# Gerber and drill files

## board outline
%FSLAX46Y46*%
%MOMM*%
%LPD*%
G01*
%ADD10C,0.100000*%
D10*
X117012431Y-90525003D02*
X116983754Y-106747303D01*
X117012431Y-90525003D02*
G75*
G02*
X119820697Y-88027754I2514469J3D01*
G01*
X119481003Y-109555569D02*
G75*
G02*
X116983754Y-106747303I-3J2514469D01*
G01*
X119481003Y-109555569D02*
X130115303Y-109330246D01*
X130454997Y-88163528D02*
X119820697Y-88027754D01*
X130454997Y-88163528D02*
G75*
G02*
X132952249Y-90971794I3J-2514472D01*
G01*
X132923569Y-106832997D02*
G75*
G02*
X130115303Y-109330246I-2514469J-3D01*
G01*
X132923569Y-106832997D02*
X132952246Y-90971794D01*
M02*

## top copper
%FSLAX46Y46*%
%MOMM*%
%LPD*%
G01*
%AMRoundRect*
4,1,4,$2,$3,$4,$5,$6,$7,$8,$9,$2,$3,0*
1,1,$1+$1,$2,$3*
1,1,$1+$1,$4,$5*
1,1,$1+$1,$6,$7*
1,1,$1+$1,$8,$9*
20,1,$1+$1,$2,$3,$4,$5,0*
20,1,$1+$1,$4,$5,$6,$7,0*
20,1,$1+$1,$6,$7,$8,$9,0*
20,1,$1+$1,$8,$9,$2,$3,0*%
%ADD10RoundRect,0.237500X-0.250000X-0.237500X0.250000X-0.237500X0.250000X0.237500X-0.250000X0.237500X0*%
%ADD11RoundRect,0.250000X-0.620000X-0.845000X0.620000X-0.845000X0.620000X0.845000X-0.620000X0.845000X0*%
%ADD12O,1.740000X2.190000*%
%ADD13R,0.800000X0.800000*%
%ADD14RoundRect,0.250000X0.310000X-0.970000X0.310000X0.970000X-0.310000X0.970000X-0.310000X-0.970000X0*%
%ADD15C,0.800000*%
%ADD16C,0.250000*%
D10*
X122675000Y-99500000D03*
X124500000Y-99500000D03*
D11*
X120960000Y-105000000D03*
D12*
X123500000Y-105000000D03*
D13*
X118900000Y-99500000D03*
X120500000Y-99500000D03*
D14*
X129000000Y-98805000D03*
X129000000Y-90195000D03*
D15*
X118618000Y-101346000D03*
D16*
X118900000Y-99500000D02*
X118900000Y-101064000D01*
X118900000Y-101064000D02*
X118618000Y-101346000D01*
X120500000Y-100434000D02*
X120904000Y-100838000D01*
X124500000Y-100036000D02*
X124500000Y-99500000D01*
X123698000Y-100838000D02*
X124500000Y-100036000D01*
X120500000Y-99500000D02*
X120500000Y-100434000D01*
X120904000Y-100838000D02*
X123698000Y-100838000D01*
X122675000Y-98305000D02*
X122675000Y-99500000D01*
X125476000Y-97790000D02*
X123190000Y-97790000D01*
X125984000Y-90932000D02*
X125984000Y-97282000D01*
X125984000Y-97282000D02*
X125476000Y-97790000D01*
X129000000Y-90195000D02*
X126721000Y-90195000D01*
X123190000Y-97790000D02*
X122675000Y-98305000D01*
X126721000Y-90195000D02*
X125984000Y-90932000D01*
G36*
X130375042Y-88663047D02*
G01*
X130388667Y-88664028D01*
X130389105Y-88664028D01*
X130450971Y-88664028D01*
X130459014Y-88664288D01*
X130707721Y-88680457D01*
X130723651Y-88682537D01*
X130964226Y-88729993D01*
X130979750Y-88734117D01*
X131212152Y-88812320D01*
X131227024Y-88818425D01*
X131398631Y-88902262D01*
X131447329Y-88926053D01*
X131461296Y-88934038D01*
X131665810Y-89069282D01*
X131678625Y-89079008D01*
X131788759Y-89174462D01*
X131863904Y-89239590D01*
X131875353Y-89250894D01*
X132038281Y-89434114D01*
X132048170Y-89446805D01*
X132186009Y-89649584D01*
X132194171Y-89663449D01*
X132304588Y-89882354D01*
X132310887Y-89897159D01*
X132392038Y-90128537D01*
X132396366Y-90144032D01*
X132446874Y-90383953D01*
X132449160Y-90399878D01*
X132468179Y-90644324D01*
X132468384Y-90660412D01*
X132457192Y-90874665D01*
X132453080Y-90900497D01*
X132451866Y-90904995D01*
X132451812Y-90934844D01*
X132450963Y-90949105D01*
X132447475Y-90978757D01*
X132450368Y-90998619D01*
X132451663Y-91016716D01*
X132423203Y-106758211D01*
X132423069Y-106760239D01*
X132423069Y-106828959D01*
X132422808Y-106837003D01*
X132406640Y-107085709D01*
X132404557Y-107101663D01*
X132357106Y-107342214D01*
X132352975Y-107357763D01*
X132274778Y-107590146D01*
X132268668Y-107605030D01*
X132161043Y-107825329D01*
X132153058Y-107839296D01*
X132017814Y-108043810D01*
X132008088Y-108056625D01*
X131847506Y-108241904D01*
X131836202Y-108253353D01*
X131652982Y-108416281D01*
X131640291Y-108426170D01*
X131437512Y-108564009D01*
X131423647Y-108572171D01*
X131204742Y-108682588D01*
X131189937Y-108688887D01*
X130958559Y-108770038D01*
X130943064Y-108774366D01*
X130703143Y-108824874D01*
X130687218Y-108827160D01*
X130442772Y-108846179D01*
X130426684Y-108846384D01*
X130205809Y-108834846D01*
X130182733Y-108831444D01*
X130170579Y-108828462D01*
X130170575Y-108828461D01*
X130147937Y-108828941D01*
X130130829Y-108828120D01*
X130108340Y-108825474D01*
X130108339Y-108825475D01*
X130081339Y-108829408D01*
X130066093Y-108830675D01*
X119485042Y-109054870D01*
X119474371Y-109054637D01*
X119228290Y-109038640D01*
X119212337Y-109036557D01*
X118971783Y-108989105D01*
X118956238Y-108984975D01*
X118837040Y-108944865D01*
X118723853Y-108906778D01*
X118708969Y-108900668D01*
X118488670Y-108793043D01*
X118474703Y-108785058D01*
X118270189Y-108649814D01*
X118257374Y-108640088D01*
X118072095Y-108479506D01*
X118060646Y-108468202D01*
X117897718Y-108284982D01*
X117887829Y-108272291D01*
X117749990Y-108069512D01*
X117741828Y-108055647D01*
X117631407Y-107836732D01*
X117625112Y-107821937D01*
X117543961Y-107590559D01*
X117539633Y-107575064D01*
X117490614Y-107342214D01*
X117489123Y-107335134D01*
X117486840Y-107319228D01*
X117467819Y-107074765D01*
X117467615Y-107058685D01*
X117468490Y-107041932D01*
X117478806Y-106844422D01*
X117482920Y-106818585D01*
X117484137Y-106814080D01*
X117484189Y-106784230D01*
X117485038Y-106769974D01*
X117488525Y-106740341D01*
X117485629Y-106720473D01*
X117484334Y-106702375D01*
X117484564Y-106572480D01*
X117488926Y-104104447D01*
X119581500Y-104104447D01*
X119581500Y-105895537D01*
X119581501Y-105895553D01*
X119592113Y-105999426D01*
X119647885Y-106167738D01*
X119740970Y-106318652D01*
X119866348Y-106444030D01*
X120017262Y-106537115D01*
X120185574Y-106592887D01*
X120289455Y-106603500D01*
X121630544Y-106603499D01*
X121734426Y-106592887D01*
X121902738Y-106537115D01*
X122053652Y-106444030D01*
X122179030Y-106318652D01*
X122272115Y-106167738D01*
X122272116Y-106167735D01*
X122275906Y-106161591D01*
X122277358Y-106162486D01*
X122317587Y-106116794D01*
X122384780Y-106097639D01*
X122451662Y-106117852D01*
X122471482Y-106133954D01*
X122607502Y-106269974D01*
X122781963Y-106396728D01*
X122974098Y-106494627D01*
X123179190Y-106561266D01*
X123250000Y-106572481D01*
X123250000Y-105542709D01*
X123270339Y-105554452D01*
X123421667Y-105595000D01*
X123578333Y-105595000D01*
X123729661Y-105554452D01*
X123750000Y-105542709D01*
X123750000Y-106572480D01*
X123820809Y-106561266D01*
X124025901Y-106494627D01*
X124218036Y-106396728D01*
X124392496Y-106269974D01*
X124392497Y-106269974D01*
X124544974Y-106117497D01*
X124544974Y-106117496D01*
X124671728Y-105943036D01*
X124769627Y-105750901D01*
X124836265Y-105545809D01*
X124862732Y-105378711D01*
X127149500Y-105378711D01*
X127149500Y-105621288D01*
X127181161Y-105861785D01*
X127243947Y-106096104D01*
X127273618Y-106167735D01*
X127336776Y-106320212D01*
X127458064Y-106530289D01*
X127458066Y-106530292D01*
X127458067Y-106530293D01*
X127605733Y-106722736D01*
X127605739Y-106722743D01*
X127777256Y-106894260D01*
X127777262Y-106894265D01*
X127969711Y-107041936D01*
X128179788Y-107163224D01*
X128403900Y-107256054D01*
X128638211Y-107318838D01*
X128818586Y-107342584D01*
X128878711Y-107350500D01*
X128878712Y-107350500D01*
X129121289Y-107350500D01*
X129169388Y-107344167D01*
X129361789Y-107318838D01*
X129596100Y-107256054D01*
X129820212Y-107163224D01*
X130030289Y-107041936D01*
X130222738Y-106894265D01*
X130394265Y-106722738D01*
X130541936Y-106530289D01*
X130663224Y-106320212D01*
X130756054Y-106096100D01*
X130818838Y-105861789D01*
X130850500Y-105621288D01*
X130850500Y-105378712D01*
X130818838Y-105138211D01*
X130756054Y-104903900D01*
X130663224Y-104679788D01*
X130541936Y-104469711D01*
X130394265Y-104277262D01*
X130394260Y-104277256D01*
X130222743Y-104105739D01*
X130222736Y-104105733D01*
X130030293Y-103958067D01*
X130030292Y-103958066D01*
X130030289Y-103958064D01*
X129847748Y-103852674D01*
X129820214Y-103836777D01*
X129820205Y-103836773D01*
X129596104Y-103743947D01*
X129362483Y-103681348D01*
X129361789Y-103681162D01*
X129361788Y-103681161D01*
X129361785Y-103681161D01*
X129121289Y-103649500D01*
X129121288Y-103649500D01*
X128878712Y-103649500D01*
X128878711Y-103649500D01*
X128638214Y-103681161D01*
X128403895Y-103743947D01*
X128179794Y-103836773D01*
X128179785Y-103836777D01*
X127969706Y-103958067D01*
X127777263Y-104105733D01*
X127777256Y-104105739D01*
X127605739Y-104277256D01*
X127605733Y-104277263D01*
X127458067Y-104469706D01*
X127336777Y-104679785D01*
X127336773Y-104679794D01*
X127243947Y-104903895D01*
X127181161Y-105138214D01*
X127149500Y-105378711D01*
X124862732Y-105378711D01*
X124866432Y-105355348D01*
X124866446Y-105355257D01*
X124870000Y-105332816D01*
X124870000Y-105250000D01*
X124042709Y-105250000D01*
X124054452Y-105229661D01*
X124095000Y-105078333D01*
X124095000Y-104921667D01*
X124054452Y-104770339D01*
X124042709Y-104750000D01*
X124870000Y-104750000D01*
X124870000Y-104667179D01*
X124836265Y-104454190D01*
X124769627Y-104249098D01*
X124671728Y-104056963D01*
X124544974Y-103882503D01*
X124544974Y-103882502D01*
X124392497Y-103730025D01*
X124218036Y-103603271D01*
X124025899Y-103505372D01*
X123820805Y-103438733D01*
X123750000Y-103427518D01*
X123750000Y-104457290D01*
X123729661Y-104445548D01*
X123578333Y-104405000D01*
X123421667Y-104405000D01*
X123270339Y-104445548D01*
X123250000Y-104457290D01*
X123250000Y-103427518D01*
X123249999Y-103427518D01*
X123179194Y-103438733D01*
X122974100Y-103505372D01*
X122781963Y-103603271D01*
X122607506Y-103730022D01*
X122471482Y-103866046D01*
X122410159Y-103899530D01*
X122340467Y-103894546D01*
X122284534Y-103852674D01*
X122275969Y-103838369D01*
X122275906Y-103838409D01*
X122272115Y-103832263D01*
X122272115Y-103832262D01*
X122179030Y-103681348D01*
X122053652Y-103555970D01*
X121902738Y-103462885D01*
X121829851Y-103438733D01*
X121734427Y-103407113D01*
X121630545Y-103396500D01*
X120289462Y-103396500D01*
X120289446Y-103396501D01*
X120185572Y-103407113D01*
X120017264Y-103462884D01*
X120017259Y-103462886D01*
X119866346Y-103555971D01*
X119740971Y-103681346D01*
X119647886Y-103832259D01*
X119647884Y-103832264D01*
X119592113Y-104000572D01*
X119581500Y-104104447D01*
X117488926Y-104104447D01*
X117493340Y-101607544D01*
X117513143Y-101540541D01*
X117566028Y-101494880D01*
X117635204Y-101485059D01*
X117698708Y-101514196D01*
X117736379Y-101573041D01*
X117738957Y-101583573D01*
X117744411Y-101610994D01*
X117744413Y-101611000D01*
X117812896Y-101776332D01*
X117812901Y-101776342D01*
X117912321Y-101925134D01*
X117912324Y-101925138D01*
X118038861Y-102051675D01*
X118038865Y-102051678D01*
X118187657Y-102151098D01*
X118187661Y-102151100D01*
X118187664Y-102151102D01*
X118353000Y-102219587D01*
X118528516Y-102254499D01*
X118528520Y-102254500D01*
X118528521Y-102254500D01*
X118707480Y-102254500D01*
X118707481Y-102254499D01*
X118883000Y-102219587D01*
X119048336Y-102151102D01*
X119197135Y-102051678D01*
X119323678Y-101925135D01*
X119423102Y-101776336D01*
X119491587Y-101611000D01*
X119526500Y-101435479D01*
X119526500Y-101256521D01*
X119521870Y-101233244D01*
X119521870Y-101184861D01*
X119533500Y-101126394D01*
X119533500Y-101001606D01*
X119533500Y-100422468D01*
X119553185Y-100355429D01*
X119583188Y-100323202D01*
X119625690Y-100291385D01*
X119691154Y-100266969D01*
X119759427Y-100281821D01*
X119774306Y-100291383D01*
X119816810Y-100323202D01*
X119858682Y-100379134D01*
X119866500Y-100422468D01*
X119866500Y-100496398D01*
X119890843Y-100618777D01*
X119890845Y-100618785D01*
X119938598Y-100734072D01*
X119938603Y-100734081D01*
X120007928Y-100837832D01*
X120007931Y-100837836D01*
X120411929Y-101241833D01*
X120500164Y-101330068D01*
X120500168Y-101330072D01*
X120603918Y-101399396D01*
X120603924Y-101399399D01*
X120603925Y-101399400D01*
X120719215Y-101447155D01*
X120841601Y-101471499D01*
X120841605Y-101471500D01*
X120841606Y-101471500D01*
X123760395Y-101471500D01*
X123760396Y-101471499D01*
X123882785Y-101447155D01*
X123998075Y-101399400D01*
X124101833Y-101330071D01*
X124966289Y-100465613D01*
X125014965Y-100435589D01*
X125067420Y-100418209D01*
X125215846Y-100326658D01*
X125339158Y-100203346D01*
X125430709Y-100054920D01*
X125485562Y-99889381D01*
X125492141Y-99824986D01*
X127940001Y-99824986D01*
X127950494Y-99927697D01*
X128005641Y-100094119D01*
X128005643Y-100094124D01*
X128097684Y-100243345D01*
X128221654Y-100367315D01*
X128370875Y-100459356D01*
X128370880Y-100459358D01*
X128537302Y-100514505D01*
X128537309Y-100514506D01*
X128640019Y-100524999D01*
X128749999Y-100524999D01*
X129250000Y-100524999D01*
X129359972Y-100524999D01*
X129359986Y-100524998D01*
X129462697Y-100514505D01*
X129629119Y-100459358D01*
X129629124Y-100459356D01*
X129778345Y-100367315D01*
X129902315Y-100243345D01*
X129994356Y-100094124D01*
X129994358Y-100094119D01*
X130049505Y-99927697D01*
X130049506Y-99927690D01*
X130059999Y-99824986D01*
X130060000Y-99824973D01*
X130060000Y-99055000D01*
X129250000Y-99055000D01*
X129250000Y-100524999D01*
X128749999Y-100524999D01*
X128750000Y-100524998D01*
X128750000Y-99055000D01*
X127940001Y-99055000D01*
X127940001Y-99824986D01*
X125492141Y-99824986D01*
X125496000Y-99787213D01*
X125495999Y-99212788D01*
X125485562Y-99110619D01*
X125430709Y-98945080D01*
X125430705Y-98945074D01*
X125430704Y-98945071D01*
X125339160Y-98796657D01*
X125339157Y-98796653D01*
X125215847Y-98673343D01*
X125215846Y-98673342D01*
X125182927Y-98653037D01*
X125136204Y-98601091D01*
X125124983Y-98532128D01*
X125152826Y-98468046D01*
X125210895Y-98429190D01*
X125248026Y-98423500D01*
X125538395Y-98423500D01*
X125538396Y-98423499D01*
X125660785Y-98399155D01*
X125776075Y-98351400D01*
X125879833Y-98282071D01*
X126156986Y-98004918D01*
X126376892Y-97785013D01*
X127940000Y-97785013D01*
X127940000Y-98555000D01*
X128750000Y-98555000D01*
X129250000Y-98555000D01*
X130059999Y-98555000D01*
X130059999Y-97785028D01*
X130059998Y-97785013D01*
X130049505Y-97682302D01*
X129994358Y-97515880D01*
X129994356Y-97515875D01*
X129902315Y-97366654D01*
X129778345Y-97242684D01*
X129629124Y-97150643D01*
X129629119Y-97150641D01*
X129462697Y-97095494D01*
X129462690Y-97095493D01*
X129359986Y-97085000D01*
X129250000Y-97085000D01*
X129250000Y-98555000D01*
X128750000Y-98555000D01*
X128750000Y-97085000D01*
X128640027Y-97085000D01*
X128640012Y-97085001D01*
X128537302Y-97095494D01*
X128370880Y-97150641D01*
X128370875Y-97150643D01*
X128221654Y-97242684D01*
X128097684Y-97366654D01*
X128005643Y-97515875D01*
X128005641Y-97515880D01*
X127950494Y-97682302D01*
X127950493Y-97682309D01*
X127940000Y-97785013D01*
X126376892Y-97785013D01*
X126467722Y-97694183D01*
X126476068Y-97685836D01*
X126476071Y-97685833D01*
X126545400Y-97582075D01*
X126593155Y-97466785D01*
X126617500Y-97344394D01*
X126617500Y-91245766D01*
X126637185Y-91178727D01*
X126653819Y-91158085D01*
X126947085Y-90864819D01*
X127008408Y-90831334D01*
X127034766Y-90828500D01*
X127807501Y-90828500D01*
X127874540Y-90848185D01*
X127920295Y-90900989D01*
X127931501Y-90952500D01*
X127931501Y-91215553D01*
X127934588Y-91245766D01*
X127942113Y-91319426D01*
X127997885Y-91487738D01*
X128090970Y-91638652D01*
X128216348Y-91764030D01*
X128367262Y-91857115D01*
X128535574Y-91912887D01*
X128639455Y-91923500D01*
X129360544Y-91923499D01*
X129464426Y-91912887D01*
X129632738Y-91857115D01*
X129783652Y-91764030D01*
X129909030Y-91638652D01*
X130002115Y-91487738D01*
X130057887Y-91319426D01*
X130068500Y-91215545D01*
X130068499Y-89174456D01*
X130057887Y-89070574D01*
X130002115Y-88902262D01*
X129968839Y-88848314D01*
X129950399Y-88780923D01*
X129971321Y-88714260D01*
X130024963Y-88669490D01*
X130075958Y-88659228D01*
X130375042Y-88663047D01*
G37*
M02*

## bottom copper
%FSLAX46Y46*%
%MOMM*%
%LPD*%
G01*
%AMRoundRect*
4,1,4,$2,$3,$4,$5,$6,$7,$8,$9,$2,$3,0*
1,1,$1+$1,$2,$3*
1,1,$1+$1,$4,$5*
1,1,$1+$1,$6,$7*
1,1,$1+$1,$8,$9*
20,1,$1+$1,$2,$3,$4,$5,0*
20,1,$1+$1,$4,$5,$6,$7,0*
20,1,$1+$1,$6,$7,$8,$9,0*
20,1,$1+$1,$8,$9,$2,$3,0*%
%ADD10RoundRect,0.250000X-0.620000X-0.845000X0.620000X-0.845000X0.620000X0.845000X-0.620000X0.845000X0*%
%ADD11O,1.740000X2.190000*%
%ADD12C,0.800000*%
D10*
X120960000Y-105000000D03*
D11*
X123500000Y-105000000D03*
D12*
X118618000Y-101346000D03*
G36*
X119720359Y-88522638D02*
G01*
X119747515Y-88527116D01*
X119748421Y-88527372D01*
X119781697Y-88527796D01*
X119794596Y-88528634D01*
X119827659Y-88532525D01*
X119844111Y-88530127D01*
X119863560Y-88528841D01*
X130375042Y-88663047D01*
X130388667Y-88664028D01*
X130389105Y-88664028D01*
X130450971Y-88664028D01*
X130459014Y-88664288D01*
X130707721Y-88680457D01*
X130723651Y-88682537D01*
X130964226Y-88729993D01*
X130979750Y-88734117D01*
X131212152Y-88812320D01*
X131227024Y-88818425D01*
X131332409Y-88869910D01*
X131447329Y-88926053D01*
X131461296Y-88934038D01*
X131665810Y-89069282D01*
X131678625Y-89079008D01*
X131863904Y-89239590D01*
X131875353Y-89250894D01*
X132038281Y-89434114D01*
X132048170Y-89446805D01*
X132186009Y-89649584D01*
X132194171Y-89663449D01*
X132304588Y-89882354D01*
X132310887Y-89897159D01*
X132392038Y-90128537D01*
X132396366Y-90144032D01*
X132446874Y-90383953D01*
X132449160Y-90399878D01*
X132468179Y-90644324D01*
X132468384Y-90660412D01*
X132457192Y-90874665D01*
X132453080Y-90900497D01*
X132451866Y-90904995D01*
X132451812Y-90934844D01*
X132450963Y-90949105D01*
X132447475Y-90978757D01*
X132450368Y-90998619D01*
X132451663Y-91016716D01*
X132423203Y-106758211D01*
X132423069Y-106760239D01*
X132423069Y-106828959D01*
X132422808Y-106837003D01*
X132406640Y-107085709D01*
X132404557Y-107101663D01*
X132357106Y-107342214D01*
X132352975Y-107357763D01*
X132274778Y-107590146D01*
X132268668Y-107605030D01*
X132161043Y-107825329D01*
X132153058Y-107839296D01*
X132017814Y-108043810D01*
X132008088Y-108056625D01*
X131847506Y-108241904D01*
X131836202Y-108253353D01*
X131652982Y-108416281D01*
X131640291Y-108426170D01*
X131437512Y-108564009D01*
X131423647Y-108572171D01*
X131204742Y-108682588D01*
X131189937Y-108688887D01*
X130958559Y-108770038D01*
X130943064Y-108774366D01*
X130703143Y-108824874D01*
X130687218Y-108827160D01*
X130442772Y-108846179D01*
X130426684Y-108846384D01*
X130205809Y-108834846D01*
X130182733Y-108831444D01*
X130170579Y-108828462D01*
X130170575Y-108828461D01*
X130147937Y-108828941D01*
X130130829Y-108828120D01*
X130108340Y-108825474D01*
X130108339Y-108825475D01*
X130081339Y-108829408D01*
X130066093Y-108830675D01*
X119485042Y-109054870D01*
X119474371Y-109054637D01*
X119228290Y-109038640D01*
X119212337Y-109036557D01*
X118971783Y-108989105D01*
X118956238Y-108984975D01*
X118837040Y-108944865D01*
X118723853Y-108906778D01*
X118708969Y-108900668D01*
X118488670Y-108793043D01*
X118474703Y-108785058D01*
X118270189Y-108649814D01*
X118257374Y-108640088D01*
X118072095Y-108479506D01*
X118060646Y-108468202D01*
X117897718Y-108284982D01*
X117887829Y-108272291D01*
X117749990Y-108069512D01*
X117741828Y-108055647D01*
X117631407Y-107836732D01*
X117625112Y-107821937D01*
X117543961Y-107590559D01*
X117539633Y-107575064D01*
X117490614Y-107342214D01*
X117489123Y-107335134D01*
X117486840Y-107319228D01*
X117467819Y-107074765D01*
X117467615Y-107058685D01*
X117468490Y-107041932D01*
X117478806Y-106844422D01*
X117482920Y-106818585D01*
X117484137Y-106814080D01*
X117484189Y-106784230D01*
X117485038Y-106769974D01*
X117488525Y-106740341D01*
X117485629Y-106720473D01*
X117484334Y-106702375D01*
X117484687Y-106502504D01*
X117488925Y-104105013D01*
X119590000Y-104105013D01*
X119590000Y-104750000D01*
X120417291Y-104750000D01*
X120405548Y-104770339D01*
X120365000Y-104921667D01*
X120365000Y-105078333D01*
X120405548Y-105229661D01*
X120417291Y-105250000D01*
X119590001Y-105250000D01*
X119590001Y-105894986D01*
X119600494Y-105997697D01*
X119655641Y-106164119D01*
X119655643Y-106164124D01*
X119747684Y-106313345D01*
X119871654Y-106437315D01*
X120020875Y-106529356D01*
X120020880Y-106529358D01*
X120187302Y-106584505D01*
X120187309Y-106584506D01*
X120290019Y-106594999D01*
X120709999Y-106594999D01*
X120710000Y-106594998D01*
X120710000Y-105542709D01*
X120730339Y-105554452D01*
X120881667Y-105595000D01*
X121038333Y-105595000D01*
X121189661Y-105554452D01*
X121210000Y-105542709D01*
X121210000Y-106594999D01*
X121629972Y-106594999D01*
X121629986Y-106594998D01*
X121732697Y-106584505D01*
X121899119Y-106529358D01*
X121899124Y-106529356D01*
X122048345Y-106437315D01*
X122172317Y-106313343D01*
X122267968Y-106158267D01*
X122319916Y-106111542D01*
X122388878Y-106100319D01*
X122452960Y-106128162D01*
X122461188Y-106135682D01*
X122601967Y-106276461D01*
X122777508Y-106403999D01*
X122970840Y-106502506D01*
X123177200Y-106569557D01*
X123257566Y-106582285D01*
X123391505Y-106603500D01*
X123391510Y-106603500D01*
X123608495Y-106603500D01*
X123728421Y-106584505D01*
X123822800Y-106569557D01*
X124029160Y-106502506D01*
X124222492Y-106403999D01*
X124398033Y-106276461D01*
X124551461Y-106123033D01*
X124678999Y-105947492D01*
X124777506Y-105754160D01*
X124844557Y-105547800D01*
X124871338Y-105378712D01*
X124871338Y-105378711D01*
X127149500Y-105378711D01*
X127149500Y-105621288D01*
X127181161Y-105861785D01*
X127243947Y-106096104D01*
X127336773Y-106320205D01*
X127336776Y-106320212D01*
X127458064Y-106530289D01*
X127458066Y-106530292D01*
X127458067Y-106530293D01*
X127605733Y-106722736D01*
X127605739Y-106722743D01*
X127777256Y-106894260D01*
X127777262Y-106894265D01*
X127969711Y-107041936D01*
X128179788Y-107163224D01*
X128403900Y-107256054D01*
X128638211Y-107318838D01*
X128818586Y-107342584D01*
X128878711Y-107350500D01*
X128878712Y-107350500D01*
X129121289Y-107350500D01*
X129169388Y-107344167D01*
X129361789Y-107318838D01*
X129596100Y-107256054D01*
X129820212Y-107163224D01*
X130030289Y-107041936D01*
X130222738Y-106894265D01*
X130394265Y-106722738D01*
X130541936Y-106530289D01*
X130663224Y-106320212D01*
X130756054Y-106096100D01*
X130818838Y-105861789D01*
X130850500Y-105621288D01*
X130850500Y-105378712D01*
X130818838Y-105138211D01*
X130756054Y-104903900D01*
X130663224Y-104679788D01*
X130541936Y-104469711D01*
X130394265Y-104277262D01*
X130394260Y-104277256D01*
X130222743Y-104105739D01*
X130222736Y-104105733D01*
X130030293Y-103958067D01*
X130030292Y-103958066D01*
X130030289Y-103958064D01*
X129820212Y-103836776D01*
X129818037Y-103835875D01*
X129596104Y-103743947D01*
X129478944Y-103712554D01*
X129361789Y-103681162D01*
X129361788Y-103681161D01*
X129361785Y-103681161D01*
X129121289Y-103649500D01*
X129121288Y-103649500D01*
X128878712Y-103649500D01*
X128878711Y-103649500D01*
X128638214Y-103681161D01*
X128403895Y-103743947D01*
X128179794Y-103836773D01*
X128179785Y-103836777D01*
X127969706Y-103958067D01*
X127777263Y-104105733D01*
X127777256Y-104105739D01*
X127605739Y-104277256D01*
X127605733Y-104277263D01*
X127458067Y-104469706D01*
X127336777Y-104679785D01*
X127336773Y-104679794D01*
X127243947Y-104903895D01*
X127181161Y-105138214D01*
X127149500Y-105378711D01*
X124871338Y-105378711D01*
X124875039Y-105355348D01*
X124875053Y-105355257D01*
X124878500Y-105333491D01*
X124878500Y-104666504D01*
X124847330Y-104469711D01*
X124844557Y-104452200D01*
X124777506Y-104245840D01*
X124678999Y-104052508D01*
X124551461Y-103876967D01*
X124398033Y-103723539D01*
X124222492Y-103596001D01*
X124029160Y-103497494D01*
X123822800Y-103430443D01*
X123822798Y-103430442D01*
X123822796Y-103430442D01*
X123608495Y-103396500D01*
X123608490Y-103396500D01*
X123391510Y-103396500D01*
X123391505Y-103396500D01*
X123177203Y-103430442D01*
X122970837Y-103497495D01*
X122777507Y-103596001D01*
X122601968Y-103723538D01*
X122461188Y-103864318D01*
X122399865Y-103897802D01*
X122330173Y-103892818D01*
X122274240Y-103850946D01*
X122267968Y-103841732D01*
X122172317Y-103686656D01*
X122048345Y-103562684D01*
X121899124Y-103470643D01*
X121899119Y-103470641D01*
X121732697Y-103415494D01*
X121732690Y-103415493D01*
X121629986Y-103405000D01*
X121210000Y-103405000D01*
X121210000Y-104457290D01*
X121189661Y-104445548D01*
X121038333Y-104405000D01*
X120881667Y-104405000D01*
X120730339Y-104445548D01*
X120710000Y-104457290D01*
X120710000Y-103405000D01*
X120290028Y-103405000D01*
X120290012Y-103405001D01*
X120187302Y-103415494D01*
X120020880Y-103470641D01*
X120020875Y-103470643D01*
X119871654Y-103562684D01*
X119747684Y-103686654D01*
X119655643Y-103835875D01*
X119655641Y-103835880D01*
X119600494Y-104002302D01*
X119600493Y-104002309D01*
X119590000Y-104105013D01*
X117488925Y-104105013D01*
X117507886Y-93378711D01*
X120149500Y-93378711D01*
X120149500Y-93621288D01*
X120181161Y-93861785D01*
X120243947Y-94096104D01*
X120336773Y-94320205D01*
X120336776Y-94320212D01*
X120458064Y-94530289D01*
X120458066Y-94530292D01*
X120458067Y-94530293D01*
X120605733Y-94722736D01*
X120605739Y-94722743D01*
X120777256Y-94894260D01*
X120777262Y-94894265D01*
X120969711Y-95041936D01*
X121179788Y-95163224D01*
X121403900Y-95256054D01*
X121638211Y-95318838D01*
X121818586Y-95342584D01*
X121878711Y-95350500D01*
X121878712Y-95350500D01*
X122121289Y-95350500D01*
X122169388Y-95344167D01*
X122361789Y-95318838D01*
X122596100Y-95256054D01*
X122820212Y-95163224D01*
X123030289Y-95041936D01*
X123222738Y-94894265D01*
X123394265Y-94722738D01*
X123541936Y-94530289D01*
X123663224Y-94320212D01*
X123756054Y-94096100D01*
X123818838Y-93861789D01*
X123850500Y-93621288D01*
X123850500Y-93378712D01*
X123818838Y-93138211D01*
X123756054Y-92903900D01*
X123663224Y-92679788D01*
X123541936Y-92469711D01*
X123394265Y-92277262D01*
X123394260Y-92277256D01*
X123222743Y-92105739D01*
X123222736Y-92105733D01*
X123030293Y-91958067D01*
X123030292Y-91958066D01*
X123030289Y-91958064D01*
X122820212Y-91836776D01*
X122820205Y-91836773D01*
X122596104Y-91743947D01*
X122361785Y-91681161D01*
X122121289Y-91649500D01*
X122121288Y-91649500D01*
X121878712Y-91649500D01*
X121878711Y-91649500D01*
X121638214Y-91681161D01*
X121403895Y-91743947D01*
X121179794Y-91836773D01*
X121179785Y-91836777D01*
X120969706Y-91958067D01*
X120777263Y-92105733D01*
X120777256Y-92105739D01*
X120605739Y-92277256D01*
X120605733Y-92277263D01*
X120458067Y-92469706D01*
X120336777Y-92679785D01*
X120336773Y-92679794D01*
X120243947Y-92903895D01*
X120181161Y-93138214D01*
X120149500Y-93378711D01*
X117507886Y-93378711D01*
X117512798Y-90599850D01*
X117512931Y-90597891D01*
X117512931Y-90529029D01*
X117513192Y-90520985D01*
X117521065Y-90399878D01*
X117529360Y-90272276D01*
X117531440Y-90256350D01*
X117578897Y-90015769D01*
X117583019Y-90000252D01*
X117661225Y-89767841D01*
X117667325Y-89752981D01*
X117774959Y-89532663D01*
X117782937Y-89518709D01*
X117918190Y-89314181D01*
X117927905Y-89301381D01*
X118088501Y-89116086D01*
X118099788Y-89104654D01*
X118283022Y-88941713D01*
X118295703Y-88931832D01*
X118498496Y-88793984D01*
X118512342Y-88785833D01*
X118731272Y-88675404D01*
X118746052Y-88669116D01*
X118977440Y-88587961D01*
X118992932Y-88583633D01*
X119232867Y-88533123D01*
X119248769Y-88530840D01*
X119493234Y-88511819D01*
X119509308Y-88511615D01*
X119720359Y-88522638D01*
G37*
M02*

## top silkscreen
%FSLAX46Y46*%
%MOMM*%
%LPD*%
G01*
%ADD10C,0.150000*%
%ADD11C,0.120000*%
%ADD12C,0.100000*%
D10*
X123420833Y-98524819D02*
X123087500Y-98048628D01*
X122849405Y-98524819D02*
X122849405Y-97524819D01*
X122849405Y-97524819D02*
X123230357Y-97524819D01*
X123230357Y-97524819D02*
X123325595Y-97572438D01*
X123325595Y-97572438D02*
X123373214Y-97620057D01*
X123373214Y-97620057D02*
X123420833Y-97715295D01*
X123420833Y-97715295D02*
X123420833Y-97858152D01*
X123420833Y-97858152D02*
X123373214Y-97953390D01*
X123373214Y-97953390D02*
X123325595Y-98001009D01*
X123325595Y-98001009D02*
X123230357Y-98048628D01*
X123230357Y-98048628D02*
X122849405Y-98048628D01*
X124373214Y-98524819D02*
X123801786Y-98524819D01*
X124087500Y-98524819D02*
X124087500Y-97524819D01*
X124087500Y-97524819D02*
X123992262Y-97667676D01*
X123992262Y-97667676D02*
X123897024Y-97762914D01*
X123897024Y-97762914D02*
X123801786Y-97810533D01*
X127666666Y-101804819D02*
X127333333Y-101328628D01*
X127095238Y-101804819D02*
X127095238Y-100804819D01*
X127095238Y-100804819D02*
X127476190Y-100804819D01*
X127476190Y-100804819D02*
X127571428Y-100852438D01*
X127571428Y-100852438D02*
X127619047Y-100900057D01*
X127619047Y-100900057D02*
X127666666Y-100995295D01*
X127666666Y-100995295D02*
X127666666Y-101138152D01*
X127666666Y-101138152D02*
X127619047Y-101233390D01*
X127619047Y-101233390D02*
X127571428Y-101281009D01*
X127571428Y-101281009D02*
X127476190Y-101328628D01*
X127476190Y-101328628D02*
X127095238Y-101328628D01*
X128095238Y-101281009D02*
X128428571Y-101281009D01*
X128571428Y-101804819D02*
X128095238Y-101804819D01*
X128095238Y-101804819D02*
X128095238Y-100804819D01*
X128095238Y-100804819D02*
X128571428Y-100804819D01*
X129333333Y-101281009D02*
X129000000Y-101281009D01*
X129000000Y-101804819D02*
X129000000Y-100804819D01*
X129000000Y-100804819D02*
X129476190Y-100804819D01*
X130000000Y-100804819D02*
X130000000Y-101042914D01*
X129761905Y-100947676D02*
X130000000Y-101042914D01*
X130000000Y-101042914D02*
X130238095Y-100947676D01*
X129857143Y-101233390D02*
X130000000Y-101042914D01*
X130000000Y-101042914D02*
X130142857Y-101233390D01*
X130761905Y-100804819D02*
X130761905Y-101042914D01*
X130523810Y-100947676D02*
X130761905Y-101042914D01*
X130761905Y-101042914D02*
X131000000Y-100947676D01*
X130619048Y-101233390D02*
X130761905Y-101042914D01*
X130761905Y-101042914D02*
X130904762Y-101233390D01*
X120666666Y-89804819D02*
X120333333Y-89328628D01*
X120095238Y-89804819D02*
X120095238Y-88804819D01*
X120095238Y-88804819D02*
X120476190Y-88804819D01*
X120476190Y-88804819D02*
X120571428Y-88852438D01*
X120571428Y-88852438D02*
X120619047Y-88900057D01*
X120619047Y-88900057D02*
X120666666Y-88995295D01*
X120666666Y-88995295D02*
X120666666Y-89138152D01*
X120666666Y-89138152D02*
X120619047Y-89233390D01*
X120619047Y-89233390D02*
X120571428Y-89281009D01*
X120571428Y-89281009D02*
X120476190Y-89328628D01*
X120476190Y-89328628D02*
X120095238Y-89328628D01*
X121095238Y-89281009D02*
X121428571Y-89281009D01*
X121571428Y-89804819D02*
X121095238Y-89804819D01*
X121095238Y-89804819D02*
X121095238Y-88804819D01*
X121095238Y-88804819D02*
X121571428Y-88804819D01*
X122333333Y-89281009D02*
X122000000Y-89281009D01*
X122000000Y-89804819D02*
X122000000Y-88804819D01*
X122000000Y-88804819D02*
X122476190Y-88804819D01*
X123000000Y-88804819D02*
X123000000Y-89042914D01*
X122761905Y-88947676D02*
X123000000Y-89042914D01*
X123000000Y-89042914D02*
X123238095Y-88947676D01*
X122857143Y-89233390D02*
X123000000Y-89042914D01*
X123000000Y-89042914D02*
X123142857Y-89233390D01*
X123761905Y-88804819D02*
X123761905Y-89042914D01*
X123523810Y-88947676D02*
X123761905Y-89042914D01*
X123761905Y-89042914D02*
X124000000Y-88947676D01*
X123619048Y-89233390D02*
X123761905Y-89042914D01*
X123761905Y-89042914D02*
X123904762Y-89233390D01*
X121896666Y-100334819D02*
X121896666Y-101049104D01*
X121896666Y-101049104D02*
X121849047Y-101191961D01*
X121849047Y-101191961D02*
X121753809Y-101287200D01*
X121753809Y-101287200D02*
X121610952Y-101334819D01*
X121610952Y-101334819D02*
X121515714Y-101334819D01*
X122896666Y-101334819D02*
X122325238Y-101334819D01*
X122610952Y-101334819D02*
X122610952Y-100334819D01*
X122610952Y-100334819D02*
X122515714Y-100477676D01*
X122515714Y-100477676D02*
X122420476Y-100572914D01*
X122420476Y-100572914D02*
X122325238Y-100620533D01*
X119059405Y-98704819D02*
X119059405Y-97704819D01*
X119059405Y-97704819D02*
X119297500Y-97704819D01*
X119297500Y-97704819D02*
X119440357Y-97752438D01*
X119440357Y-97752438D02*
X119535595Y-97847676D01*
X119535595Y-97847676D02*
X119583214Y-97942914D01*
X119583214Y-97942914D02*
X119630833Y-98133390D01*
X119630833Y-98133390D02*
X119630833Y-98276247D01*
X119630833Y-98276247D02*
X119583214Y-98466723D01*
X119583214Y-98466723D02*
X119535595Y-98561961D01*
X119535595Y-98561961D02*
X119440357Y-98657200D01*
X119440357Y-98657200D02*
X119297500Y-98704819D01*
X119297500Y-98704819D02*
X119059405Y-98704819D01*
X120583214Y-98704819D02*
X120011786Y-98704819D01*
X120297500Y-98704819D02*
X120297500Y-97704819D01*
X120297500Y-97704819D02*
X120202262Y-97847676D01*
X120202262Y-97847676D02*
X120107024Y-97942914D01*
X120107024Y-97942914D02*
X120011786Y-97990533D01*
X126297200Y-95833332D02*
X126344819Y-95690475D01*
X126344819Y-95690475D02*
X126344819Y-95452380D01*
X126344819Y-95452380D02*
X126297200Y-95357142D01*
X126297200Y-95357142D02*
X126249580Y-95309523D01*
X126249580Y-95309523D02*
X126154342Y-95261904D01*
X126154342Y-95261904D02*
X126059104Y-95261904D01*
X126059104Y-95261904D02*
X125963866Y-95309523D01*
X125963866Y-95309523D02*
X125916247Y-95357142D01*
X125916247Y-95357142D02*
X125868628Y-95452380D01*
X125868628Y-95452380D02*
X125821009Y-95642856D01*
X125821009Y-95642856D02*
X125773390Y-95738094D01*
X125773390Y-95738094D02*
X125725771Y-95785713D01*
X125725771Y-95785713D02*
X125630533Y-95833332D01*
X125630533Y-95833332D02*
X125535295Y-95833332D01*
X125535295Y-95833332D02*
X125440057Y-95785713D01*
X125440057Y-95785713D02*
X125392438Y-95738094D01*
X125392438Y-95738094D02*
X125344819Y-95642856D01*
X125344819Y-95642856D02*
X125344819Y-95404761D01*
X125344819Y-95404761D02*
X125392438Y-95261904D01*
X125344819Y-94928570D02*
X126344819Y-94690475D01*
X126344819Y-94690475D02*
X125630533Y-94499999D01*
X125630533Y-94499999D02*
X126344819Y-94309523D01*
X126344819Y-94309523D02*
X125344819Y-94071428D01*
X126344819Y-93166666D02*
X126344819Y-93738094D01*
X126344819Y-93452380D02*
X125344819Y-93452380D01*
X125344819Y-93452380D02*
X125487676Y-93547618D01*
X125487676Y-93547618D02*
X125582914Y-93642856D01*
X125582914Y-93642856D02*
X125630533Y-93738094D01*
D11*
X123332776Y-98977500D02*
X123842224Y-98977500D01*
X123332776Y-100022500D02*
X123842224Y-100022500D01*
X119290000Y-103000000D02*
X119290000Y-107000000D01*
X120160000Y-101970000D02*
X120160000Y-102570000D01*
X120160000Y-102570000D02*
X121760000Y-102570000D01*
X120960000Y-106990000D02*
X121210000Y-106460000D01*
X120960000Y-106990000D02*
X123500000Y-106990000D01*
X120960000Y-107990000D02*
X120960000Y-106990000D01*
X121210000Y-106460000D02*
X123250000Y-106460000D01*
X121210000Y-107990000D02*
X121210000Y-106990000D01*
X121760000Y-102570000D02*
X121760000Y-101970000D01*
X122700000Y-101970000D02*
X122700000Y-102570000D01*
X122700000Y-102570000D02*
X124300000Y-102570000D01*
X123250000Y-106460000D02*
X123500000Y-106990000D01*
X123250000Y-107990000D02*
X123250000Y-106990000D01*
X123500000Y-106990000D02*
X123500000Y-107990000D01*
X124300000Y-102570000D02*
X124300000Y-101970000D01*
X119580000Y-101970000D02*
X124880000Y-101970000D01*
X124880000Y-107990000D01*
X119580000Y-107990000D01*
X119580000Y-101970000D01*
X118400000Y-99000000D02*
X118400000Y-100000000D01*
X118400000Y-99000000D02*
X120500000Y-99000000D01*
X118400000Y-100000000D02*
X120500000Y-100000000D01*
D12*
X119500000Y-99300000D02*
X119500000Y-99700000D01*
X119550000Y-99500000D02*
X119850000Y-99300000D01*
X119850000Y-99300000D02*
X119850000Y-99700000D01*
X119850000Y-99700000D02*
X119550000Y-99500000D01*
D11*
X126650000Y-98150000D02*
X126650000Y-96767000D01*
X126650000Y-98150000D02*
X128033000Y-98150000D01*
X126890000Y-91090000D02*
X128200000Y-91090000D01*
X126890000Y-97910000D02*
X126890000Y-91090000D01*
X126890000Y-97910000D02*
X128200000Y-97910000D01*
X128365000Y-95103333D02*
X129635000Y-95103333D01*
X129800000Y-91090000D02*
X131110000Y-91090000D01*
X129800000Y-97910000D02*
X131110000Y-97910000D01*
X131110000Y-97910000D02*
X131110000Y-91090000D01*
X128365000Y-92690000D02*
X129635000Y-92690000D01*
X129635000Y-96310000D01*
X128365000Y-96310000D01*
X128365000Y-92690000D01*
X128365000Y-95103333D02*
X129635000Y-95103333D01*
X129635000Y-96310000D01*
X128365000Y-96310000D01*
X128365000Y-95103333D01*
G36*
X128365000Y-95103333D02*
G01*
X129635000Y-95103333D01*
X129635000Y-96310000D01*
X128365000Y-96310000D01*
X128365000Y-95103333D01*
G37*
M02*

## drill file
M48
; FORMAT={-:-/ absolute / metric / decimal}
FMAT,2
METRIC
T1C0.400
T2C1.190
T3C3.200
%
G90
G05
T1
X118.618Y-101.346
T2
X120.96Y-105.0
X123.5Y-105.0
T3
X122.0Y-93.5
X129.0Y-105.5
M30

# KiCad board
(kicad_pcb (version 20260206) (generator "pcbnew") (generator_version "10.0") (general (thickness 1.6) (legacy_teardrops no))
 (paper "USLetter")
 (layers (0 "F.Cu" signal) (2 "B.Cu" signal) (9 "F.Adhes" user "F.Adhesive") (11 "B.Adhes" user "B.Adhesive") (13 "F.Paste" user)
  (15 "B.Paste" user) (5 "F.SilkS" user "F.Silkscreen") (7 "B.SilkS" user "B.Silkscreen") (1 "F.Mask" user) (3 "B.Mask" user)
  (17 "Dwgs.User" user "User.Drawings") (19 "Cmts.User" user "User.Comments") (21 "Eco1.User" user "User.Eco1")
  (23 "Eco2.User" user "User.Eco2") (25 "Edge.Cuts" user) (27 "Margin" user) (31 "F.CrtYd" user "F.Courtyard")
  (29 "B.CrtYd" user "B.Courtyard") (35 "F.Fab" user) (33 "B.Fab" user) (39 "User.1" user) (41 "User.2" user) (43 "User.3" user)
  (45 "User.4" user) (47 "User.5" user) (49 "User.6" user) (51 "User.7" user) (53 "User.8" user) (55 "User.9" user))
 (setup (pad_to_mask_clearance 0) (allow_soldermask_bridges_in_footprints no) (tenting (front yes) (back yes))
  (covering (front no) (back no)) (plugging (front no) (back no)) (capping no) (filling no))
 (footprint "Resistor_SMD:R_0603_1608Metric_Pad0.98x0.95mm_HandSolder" (layer "F.Cu") (at 123.5875 99.5)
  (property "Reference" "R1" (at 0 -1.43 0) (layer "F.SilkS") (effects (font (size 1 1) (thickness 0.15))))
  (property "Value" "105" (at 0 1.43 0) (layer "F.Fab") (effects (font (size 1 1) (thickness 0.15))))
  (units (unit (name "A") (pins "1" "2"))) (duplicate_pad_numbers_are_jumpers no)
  (fp_line (start -0.254724 -0.5225) (end 0.254724 -0.5225) (stroke (width 0.12) (type solid)) (layer "F.SilkS"))
  (fp_line (start -0.254724 0.5225) (end 0.254724 0.5225) (stroke (width 0.12) (type solid)) (layer "F.SilkS"))
  (pad "1" smd roundrect (at -0.9125 0) (size 0.975 0.95) (layers "F.Cu" "F.Mask" "F.Paste") (roundrect_rratio 0.25) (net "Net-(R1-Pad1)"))
  (pad "2" smd roundrect (at 0.9125 0) (size 0.975 0.95) (layers "F.Cu" "F.Mask" "F.Paste") (roundrect_rratio 0.25) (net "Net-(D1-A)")))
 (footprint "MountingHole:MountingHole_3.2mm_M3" (layer "F.Cu") (at 129 105.5)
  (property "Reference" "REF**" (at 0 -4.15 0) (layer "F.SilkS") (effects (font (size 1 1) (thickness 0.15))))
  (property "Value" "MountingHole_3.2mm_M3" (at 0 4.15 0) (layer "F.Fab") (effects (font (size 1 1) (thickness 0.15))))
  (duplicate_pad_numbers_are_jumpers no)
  (pad "" np_thru_hole circle (at 0 0) (size 3.2 3.2) (drill 3.2) (layers "*.Cu" "*.Mask")))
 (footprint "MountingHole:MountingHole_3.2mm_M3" (layer "F.Cu") (at 122 93.5)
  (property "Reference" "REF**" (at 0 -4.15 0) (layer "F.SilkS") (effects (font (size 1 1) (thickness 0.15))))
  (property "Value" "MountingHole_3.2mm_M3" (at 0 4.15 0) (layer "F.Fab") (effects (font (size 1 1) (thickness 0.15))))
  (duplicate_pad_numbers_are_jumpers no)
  (pad "" np_thru_hole circle (at 0 0) (size 3.2 3.2) (drill 3.2) (layers "*.Cu" "*.Mask")))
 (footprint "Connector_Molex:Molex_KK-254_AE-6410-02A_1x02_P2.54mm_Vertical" (layer "F.Cu") (at 120.96 105)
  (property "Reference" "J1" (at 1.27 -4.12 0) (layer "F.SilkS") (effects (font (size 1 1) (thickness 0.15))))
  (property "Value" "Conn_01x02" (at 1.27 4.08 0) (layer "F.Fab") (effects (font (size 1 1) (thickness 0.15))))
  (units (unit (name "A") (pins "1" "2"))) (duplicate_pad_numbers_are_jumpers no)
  (fp_line (start -1.67 -2) (end -1.67 2) (stroke (width 0.12) (type solid)) (layer "F.SilkS"))
  (fp_line (start -0.8 -3.03) (end -0.8 -2.43) (stroke (width 0.12) (type solid)) (layer "F.SilkS"))
  (fp_line (start -0.8 -2.43) (end 0.8 -2.43) (stroke (width 0.12) (type solid)) (layer "F.SilkS"))
  (fp_line (start 0 1.99) (end 0.25 1.46) (stroke (width 0.12) (type solid)) (layer "F.SilkS"))
  (fp_line (start 0 1.99) (end 2.54 1.99) (stroke (width 0.12) (type solid)) (layer "F.SilkS"))
  (fp_line (start 0 2.99) (end 0 1.99) (stroke (width 0.12) (type solid)) (layer "F.SilkS"))
  (fp_line (start 0.25 1.46) (end 2.29 1.46) (stroke (width 0.12) (type solid)) (layer "F.SilkS"))
  (fp_line (start 0.25 2.99) (end 0.25 1.99) (stroke (width 0.12) (type solid)) (layer "F.SilkS"))
  (fp_line (start 0.8 -2.43) (end 0.8 -3.03) (stroke (width 0.12) (type solid)) (layer "F.SilkS"))
  (fp_line (start 1.74 -3.03) (end 1.74 -2.43) (stroke (width 0.12) (type solid)) (layer "F.SilkS"))
  (fp_line (start 1.74 -2.43) (end 3.34 -2.43) (stroke (width 0.12) (type solid)) (layer "F.SilkS"))
  (fp_line (start 2.29 1.46) (end 2.54 1.99) (stroke (width 0.12) (type solid)) (layer "F.SilkS"))
  (fp_line (start 2.29 2.99) (end 2.29 1.99) (stroke (width 0.12) (type solid)) (layer "F.SilkS"))
  (fp_line (start 2.54 1.99) (end 2.54 2.99) (stroke (width 0.12) (type solid)) (layer "F.SilkS"))
  (fp_line (start 3.34 -2.43) (end 3.34 -3.03) (stroke (width 0.12) (type solid)) (layer "F.SilkS"))
  (fp_rect (start -1.38 -3.03) (end 3.92 2.99) (stroke (width 0.12) (type solid)) (fill no) (layer "F.SilkS"))
  (pad "1" thru_hole roundrect (at 0 0) (size 1.74 2.19) (drill 1.19) (layers "*.Cu" "*.Mask") (remove_unused_layers no)
   (roundrect_rratio 0.143678) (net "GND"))
  (pad "2" thru_hole oval (at 2.54 0) (size 1.74 2.19) (drill 1.19) (layers "*.Cu" "*.Mask") (remove_unused_layers no) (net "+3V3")))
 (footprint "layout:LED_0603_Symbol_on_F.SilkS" (layer "F.Cu") (at 119.7 99.5)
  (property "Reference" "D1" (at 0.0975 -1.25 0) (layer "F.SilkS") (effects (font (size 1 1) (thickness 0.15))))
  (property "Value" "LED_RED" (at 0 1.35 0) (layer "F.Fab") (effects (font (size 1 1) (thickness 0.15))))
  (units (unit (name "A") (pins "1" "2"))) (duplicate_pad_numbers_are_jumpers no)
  (fp_line (start -1.3 -0.5) (end -1.3 0.5) (stroke (width 0.12) (type solid)) (layer "F.SilkS"))
  (fp_line (start -1.3 -0.5) (end 0.8 -0.5) (stroke (width 0.12) (type solid)) (layer "F.SilkS"))
  (fp_line (start -1.3 0.5) (end 0.8 0.5) (stroke (width 0.12) (type solid)) (layer "F.SilkS"))
  (fp_line (start -0.2 -0.2) (end -0.2 0.2) (stroke (width 0.1) (type solid)) (layer "F.SilkS"))
  (fp_line (start -0.15 0) (end 0.15 -0.2) (stroke (width 0.1) (type solid)) (layer "F.SilkS"))
  (fp_line (start 0.15 -0.2) (end 0.15 0.2) (stroke (width 0.1) (type solid)) (layer "F.SilkS"))
  (fp_line (start 0.15 0.2) (end -0.15 0) (stroke (width 0.1) (type solid)) (layer "F.SilkS"))
  (pad "1" smd rect (at -0.8 0 180) (size 0.8 0.8) (layers "F.Cu" "F.Mask" "F.Paste") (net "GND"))
  (pad "2" smd rect (at 0.8 0 180) (size 0.8 0.8) (layers "F.Cu" "F.Mask" "F.Paste") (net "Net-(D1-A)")))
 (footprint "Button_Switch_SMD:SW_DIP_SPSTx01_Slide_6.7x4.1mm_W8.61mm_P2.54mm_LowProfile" (layer "F.Cu") (at 129 94.5 90)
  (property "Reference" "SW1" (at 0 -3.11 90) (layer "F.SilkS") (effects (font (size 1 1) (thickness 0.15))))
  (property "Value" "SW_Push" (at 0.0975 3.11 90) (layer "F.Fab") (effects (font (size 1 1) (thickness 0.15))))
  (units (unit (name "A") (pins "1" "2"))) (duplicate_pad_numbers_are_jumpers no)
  (fp_line (start -3.65 -2.35) (end -2.267 -2.35) (stroke (width 0.12) (type solid)) (layer "F.SilkS"))
  (fp_line (start -3.65 -2.35) (end -3.65 -0.967) (stroke (width 0.12) (type solid)) (layer "F.SilkS"))
  (fp_line (start 3.41 -2.11) (end 3.41 -0.8) (stroke (width 0.12) (type solid)) (layer "F.SilkS"))
  (fp_line (start -3.41 -2.11) (end 3.41 -2.11) (stroke (width 0.12) (type solid)) (layer "F.SilkS"))
  (fp_line (start -3.41 -2.11) (end -3.41 -0.8) (stroke (width 0.12) (type solid)) (layer "F.SilkS"))
  (fp_line (start -0.603333 -0.635) (end -0.603333 0.635) (stroke (width 0.12) (type solid)) (layer "F.SilkS"))
  (fp_line (start 3.41 0.8) (end 3.41 2.11) (stroke (width 0.12) (type solid)) (layer "F.SilkS"))
  (fp_line (start -3.41 0.8) (end -3.41 2.11) (stroke (width 0.12) (type solid)) (layer "F.SilkS"))
  (fp_line (start -3.41 2.11) (end 3.41 2.11) (stroke (width 0.12) (type solid)) (layer "F.SilkS"))
  (fp_rect (start -1.81 -0.635) (end 1.81 0.635) (stroke (width 0.12) (type solid)) (fill no) (layer "F.SilkS"))
  (fp_rect (start -1.81 -0.635) (end -0.603333 0.635) (stroke (width 0.12) (type solid)) (fill yes) (layer "F.SilkS"))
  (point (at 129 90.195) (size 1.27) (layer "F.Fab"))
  (pad "1" smd roundrect (at -4.305 0 90) (size 2.44 1.12) (layers "F.Cu" "F.Mask" "F.Paste") (roundrect_rratio 0.223214) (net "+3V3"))
  (pad "2" smd roundrect (at 4.305 0 90) (size 2.44 1.12) (layers "F.Cu" "F.Mask" "F.Paste") (roundrect_rratio 0.223214)
   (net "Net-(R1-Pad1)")))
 (gr_line (start 117.012431 90.525003) (end 116.983754 106.747303) (stroke (width 0.1) (type default)) (layer "Edge.Cuts"))
 (gr_arc (start 117.012431 90.525003) (mid 117.856 88.646) (end 119.820697 88.027754) (stroke (width 0.1) (type default))
  (layer "Edge.Cuts"))
 (gr_arc (start 119.481003 109.555569) (mid 117.602 108.712) (end 116.983754 106.747303) (stroke (width 0.1) (type default))
  (layer "Edge.Cuts"))
 (gr_line (start 119.481003 109.555569) (end 130.115303 109.330246) (stroke (width 0.1) (type default)) (layer "Edge.Cuts"))
 (gr_line (start 130.454997 88.163528) (end 119.820697 88.027754) (stroke (width 0.1) (type default)) (layer "Edge.Cuts"))
 (gr_arc (start 130.454997 88.163528) (mid 132.334 89.007097) (end 132.952246 90.971794) (stroke (width 0.1) (type default))
  (layer "Edge.Cuts"))
 (gr_arc (start 132.923569 106.832997) (mid 132.08 108.712) (end 130.115303 109.330246) (stroke (width 0.1) (type default))
  (layer "Edge.Cuts"))
 (gr_line (start 132.923569 106.832997) (end 132.952246 90.971794) (stroke (width 0.1) (type default)) (layer "Edge.Cuts"))
 (segment (start 118.9 99.5) (end 118.9 101.064) (width 0.25) (layer "F.Cu") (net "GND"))
 (segment (start 118.9 101.064) (end 118.618 101.346) (width 0.25) (layer "F.Cu") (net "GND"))
 (via (at 118.618 101.346) (size 0.8) (drill 0.4) (layers "F.Cu" "B.Cu") (free yes) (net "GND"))
 (segment (start 120.5 100.434) (end 120.904 100.838) (width 0.25) (layer "F.Cu") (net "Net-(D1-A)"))
 (segment (start 124.5 100.036) (end 124.5 99.5) (width 0.25) (layer "F.Cu") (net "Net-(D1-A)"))
 (segment (start 123.698 100.838) (end 124.5 100.036) (width 0.25) (layer "F.Cu") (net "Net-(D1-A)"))
 (segment (start 120.5 99.5) (end 120.5 100.434) (width 0.25) (layer "F.Cu") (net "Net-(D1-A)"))
 (segment (start 120.904 100.838) (end 123.698 100.838) (width 0.25) (layer "F.Cu") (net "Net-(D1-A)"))
 (segment (start 122.675 98.305) (end 122.675 99.5) (width 0.25) (layer "F.Cu") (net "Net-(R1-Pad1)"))
 (segment (start 125.476 97.79) (end 123.19 97.79) (width 0.25) (layer "F.Cu") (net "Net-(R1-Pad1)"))
 (segment (start 125.984 90.932) (end 125.984 97.282) (width 0.25) (layer "F.Cu") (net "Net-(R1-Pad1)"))
 (segment (start 125.984 97.282) (end 125.476 97.79) (width 0.25) (layer "F.Cu") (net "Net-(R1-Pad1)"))
 (segment (start 129 90.195) (end 126.721 90.195) (width 0.25) (layer "F.Cu") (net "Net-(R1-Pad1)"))
 (segment (start 123.19 97.79) (end 122.675 98.305) (width 0.25) (layer "F.Cu") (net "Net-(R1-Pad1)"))
 (segment (start 126.721 90.195) (end 125.984 90.932) (width 0.25) (layer "F.Cu") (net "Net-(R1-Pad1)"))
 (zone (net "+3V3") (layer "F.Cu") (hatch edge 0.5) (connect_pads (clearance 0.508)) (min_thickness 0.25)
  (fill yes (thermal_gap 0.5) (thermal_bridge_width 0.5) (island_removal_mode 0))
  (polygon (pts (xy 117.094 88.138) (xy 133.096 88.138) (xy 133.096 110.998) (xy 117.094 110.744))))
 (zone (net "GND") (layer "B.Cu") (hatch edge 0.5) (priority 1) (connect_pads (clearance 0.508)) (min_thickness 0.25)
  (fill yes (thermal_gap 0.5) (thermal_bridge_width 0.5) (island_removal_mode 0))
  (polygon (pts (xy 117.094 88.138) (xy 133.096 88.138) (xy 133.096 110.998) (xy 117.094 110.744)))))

